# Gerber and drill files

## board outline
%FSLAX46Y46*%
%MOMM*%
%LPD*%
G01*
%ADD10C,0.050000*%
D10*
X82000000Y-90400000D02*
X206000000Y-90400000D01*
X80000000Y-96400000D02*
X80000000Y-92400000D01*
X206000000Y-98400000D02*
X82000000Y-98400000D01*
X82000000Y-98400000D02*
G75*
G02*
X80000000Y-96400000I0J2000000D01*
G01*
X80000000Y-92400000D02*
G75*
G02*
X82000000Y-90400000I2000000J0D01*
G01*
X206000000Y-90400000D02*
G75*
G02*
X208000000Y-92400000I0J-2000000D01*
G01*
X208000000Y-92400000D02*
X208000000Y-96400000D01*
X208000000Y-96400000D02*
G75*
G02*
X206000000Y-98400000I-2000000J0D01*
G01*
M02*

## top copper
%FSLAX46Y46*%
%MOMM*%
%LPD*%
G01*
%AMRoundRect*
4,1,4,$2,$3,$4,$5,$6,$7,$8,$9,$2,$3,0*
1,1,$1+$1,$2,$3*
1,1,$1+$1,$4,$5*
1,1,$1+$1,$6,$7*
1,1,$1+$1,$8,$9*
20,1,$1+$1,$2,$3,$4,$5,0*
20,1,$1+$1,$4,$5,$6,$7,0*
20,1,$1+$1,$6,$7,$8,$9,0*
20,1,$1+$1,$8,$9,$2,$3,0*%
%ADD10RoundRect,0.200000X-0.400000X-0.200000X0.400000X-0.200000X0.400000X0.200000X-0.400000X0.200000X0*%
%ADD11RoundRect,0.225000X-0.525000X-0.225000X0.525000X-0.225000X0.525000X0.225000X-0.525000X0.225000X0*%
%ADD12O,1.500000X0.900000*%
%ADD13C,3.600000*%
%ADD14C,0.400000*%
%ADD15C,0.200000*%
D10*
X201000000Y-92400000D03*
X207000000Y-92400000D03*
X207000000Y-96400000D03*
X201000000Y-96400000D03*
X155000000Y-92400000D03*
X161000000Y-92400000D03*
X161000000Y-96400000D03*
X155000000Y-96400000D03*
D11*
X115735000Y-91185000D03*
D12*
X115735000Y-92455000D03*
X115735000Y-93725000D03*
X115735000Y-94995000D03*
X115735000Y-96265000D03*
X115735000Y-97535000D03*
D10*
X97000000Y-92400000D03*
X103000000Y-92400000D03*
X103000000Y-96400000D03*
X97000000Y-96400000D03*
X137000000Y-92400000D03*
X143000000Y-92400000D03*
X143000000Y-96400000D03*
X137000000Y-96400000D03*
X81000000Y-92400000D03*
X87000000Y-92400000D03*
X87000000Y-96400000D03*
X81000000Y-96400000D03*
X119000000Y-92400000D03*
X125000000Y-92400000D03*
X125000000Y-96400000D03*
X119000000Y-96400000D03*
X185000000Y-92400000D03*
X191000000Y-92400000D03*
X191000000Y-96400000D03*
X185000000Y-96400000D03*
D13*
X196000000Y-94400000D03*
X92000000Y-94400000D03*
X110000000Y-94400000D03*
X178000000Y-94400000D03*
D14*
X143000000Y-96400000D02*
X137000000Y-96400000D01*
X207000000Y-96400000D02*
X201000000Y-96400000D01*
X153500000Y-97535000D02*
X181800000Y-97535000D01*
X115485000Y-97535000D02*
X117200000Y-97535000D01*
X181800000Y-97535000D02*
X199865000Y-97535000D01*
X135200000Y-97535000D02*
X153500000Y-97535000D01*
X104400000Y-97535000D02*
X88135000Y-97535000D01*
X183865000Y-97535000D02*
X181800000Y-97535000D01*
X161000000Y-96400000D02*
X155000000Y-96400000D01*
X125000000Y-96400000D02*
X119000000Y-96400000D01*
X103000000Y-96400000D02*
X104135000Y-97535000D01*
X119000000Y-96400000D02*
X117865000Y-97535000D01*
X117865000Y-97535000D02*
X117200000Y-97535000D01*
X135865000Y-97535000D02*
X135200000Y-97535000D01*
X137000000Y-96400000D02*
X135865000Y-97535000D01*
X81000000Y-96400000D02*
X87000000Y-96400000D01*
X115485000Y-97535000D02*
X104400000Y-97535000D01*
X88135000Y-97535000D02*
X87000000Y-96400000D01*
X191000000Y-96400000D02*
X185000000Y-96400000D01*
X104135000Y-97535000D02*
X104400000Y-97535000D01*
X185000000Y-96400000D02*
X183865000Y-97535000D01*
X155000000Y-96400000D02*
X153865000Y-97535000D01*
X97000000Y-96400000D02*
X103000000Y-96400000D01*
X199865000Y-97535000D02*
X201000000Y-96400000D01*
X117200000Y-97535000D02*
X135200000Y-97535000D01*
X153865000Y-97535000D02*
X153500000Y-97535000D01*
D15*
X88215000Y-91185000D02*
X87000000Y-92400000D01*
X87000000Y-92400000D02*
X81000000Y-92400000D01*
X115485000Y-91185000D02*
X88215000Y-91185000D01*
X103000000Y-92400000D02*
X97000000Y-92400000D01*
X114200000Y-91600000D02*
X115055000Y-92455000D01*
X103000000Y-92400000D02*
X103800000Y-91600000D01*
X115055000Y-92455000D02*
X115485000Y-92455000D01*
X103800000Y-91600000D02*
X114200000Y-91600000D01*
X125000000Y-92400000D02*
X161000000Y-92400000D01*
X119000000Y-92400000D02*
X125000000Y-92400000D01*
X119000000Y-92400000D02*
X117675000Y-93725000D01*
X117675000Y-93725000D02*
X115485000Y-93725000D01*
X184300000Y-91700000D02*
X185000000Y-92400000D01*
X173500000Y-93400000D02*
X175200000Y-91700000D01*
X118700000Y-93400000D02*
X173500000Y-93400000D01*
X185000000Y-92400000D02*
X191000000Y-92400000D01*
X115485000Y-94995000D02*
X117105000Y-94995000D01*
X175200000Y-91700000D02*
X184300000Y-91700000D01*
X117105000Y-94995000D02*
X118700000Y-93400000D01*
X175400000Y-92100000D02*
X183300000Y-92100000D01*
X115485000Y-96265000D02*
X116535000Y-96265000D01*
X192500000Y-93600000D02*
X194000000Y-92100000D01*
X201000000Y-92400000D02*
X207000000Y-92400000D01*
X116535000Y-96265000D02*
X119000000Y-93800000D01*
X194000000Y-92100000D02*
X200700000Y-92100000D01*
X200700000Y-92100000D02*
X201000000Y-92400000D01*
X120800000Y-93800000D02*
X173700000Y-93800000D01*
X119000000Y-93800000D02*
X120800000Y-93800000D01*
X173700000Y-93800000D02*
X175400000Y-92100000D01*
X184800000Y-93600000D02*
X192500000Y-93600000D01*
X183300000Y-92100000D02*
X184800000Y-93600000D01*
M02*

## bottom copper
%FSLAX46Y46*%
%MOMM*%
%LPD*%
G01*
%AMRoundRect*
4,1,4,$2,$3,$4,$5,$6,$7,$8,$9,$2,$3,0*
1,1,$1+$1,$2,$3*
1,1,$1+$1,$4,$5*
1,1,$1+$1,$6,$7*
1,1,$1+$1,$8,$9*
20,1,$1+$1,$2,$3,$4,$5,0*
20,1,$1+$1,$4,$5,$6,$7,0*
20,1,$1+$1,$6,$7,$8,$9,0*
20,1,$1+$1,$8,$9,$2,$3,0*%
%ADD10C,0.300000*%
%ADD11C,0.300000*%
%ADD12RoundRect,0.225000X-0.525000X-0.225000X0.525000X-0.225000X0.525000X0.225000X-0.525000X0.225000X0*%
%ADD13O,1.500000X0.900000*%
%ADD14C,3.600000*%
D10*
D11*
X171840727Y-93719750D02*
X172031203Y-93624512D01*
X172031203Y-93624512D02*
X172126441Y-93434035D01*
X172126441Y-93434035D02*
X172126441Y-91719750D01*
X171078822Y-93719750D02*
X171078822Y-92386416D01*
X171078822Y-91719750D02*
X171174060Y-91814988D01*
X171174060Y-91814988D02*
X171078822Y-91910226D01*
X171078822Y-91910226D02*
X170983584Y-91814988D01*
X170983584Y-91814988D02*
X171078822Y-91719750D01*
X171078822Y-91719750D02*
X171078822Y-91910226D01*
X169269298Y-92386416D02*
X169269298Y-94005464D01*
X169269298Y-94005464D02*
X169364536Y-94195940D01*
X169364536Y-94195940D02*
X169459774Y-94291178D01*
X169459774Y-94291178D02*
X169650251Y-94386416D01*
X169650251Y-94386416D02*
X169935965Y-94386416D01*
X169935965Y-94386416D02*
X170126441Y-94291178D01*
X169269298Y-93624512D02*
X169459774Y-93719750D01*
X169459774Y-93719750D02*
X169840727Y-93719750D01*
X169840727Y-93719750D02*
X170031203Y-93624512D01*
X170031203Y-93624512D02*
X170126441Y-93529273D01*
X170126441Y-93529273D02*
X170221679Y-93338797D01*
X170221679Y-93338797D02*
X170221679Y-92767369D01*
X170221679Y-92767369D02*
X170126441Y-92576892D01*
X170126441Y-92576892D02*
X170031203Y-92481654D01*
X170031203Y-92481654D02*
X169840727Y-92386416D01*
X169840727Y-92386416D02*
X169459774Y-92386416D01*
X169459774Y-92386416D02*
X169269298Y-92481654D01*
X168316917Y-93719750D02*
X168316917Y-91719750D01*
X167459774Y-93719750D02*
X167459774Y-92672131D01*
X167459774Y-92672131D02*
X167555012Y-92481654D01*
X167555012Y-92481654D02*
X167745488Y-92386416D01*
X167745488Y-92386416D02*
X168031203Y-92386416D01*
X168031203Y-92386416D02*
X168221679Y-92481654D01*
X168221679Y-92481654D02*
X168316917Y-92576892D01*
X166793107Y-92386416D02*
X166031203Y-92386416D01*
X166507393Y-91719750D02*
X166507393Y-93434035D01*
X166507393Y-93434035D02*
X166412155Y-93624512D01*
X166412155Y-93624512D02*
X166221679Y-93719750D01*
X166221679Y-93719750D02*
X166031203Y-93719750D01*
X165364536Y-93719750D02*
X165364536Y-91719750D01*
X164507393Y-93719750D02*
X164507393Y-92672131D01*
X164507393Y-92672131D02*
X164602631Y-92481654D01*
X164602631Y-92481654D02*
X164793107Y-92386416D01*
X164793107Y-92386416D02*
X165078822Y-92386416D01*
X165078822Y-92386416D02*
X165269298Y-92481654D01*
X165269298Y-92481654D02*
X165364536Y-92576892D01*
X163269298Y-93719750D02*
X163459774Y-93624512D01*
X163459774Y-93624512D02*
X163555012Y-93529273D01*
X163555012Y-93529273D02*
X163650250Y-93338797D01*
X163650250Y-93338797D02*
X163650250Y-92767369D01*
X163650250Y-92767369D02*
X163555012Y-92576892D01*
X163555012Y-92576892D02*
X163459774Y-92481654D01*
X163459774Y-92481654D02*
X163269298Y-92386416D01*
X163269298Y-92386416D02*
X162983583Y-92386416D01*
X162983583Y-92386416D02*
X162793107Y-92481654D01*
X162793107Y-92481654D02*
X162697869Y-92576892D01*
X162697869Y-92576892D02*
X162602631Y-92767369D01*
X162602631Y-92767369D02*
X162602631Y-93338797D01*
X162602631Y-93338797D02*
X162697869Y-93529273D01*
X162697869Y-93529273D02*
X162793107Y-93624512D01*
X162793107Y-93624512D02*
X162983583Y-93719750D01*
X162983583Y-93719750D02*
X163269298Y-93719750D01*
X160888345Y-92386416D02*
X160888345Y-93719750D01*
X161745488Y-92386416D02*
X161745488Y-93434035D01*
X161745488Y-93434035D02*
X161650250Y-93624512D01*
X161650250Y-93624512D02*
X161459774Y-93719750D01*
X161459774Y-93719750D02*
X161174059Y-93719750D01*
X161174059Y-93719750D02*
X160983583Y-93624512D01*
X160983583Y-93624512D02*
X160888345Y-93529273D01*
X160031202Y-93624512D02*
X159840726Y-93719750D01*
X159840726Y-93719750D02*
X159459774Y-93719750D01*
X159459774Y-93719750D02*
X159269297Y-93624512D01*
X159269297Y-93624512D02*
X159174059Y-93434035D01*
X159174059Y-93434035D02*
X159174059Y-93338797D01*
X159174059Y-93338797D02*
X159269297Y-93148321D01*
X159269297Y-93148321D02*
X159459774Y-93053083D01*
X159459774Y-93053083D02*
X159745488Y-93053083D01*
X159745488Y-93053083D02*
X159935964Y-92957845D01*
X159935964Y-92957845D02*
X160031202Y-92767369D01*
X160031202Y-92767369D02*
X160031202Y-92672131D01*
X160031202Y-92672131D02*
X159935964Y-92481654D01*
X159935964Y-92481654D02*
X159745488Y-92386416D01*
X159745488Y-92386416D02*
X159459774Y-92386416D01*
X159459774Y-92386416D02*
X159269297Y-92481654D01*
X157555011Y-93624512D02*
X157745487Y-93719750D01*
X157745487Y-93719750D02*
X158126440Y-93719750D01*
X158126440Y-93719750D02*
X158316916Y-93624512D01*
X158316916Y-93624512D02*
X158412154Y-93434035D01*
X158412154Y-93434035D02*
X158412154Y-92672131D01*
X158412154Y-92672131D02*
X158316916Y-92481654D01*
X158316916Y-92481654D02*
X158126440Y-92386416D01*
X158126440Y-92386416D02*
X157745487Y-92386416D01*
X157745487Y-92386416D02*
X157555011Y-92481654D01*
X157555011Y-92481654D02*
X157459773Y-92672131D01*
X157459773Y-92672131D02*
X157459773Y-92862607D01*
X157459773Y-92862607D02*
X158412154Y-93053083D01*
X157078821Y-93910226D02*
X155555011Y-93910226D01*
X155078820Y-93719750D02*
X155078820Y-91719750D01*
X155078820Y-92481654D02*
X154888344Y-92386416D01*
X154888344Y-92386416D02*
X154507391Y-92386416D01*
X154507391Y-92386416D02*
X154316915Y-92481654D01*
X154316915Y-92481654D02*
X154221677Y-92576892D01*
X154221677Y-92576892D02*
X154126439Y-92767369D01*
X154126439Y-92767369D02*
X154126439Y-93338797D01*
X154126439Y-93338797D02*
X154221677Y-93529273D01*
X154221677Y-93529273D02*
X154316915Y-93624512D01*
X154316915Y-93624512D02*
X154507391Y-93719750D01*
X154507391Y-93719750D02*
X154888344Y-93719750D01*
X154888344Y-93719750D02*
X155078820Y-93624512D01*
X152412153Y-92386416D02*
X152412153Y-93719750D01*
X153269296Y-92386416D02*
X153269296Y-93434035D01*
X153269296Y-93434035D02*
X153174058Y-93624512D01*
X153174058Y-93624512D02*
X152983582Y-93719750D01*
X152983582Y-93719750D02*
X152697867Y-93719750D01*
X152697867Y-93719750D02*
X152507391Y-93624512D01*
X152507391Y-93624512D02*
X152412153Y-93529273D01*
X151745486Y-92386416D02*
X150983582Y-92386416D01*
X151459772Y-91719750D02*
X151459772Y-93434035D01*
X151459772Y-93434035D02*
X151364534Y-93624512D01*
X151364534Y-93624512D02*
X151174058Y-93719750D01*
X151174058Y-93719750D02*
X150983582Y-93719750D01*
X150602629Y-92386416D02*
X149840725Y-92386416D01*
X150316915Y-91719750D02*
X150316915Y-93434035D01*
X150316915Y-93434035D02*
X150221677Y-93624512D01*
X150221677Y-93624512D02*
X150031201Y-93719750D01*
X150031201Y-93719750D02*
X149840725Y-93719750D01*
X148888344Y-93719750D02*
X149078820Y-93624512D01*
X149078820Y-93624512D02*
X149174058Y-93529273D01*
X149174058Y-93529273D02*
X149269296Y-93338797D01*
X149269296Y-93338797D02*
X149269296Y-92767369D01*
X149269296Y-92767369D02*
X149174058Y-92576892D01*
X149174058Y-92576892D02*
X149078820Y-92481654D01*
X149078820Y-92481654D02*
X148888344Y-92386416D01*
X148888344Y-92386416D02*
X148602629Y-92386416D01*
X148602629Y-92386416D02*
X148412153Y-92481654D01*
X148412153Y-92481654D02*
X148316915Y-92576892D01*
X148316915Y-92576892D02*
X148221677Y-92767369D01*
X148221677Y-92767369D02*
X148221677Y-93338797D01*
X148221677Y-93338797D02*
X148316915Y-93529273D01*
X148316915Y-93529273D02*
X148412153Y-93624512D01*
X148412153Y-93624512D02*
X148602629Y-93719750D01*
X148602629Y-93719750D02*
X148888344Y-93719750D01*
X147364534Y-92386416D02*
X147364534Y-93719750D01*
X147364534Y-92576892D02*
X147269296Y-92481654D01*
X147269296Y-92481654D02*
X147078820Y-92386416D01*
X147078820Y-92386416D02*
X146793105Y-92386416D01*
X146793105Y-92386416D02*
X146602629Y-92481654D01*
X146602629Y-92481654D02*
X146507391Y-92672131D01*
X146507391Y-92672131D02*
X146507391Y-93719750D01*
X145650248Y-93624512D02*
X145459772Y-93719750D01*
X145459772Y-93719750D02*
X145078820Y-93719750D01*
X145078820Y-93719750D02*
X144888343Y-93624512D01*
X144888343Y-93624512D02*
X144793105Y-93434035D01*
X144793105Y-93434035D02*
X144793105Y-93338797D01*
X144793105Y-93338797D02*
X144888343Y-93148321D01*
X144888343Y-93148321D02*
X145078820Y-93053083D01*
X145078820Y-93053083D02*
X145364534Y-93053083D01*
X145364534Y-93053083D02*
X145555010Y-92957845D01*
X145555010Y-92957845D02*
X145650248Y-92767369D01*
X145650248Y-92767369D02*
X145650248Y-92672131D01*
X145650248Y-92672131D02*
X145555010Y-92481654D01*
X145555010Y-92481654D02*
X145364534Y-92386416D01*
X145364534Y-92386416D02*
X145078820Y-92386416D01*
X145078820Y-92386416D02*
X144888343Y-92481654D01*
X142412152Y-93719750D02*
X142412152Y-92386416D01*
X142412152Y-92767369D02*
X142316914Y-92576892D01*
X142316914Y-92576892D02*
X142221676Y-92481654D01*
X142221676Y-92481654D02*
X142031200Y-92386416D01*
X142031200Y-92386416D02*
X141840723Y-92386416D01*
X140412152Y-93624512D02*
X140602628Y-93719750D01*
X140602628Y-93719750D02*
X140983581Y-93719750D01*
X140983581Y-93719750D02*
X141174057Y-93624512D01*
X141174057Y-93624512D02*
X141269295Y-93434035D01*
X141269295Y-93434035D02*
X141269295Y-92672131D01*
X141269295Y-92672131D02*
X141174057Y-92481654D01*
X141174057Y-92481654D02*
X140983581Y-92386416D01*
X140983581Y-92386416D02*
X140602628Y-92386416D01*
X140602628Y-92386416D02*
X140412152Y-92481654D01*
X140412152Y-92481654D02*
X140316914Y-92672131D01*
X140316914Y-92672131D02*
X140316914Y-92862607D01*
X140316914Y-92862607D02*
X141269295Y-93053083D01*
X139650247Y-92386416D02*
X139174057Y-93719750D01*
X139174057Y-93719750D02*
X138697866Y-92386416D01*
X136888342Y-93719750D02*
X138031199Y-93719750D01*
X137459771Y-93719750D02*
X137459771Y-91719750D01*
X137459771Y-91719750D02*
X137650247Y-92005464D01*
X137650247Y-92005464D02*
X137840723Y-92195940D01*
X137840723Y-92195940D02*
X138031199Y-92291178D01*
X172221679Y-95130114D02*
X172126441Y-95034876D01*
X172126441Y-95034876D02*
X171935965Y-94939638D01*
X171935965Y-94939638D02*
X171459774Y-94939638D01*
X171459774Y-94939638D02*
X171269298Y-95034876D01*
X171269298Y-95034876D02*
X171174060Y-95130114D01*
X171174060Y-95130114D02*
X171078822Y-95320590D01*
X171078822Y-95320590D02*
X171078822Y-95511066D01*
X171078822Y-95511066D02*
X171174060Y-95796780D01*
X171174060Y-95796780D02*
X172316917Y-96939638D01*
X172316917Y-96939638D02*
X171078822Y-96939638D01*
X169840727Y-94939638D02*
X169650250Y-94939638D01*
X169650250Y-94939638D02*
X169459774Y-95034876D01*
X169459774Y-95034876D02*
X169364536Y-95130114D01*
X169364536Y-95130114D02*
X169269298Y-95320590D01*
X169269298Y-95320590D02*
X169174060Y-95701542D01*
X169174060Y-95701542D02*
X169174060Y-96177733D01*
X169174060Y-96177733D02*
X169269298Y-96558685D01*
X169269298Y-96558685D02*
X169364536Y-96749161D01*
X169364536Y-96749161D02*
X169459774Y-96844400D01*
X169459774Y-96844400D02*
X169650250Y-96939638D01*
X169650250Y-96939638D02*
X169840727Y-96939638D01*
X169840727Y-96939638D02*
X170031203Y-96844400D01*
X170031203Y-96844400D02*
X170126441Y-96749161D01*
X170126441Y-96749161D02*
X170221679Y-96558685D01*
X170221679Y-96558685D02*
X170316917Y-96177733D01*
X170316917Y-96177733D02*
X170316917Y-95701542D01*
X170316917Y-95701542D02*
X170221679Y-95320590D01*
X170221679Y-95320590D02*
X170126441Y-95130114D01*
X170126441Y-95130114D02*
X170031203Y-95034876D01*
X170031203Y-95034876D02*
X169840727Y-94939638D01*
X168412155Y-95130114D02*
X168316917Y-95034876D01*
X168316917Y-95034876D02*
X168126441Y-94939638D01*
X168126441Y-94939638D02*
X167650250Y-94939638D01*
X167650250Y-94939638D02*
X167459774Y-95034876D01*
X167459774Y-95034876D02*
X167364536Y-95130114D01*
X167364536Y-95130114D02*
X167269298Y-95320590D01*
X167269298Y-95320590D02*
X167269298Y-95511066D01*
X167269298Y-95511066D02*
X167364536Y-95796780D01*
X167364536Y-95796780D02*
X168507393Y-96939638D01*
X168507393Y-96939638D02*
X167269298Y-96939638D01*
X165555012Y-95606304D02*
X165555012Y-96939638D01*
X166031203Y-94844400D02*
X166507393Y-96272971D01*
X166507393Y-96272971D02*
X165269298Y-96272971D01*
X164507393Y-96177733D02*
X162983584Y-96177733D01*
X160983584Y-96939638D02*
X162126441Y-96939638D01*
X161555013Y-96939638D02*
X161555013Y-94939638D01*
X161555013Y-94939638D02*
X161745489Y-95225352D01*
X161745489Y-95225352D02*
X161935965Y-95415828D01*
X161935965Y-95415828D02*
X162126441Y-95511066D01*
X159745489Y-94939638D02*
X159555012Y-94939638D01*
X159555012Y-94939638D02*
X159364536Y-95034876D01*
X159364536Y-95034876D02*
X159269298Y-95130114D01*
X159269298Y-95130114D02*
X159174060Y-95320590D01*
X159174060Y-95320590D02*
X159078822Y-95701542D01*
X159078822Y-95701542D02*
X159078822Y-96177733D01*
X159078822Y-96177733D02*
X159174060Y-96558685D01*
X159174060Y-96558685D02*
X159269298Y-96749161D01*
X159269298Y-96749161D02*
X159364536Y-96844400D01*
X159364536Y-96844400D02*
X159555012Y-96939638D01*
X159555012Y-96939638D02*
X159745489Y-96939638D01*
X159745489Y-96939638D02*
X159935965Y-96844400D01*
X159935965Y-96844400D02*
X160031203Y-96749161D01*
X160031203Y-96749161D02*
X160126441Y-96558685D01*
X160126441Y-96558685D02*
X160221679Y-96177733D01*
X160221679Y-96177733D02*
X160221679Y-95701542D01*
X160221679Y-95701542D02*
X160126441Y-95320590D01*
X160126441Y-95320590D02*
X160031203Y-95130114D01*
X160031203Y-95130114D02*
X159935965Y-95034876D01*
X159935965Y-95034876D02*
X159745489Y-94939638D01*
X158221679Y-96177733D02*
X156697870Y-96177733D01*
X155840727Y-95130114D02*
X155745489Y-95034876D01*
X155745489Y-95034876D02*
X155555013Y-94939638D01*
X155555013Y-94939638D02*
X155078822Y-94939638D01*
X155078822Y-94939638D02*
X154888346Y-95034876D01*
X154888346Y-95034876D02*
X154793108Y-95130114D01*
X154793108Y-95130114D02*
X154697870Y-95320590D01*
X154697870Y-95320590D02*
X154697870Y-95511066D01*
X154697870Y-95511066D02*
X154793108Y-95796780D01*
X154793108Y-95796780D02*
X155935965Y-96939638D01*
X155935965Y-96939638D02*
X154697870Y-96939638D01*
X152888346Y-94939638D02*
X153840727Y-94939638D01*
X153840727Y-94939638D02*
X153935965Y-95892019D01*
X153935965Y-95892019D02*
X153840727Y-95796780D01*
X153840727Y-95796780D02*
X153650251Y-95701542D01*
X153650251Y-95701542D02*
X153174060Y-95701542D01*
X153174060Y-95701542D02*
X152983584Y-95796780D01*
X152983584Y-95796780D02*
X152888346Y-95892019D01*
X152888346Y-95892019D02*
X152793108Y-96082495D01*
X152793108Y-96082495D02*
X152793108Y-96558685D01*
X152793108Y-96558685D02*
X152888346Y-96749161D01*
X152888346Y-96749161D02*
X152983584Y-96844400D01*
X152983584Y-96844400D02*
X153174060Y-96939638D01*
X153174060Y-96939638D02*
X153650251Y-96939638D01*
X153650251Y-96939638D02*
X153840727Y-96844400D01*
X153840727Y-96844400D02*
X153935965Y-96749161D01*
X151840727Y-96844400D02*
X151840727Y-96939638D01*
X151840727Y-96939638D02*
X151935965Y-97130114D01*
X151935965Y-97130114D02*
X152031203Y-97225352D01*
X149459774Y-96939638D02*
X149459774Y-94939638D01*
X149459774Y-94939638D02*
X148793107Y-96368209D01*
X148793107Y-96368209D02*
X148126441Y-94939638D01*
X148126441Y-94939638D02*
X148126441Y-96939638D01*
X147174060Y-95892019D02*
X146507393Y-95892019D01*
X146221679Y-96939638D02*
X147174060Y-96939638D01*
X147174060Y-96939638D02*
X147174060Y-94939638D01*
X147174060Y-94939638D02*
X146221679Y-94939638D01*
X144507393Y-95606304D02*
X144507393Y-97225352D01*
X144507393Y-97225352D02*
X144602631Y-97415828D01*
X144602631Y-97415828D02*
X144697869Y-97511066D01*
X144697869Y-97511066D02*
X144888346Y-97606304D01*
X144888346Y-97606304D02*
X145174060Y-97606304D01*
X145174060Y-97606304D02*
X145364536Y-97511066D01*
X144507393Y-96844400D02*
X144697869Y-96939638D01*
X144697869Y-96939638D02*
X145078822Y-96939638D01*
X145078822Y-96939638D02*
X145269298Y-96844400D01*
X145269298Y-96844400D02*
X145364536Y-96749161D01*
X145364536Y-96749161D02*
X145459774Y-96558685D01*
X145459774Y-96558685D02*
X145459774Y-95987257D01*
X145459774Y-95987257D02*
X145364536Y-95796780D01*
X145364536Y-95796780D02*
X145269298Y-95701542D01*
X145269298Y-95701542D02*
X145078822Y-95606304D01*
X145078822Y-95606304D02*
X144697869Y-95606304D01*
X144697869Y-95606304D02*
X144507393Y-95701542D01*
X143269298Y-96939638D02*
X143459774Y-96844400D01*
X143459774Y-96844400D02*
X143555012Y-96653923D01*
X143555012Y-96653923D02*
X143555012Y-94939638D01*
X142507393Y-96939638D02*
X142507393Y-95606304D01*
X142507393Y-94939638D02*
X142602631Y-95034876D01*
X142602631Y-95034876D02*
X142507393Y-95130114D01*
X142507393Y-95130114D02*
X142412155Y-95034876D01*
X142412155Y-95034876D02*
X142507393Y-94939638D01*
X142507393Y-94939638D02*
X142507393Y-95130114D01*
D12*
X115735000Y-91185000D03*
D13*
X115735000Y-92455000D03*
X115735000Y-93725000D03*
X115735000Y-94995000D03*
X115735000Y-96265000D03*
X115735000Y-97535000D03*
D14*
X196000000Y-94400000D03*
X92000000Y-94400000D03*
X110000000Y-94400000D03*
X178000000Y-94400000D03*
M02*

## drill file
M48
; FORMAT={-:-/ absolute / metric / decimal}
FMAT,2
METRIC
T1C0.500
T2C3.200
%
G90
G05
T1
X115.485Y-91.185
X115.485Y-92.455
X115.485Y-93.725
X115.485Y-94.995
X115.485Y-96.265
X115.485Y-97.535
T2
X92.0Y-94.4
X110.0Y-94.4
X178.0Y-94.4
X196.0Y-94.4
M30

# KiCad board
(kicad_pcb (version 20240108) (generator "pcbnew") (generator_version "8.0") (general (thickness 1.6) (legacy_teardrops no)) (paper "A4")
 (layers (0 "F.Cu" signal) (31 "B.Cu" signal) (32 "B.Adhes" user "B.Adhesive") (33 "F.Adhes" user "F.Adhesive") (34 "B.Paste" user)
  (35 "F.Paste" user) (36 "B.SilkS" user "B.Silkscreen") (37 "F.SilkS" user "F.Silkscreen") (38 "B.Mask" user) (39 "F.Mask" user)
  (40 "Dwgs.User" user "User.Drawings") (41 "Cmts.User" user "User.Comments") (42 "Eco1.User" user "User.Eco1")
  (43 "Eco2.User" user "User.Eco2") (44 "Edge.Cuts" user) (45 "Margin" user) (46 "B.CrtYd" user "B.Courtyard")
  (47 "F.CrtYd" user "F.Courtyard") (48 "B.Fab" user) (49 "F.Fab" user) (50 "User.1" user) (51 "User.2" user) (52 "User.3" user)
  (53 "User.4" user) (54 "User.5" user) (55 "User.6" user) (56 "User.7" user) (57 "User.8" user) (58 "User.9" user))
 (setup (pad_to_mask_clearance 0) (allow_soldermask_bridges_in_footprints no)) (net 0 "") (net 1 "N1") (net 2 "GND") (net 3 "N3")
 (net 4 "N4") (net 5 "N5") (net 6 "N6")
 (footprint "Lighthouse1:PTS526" (layer "F.Cu") (at 204 94.4)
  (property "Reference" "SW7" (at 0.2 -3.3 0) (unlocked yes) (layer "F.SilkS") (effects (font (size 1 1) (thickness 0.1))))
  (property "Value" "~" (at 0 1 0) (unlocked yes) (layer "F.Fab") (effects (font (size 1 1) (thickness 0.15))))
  (pad "1" smd roundrect (at -3 -2) (size 1.2 0.8) (layers "F.Cu" "F.Paste" "F.Mask") (roundrect_rratio 0.25) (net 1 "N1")
   (thermal_bridge_angle 45))
  (pad "2" smd roundrect (at 3 -2) (size 1.2 0.8) (layers "F.Cu" "F.Paste" "F.Mask") (roundrect_rratio 0.25) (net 1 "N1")
   (thermal_bridge_angle 45))
  (pad "3" smd roundrect (at 3 2) (size 1.2 0.8) (layers "F.Cu" "F.Paste" "F.Mask") (roundrect_rratio 0.25) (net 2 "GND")
   (thermal_bridge_angle 45))
  (pad "4" smd roundrect (at -3 2) (size 1.2 0.8) (layers "F.Cu" "F.Paste" "F.Mask") (roundrect_rratio 0.25) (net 2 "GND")
   (thermal_bridge_angle 45)))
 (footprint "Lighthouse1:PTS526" (layer "F.Cu") (at 158 94.4)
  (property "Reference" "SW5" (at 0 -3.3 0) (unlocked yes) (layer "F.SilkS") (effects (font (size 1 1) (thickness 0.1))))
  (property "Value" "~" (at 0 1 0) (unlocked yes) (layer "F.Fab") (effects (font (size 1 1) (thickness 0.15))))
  (pad "1" smd roundrect (at -3 -2) (size 1.2 0.8) (layers "F.Cu" "F.Paste" "F.Mask") (roundrect_rratio 0.25) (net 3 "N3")
   (thermal_bridge_angle 45))
  (pad "2" smd roundrect (at 3 -2) (size 1.2 0.8) (layers "F.Cu" "F.Paste" "F.Mask") (roundrect_rratio 0.25) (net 3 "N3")
   (thermal_bridge_angle 45))
  (pad "3" smd roundrect (at 3 2) (size 1.2 0.8) (layers "F.Cu" "F.Paste" "F.Mask") (roundrect_rratio 0.25) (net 2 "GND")
   (thermal_bridge_angle 45))
  (pad "4" smd roundrect (at -3 2) (size 1.2 0.8) (layers "F.Cu" "F.Paste" "F.Mask") (roundrect_rratio 0.25) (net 2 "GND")
   (thermal_bridge_angle 45)))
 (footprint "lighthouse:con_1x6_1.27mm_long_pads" (layer "F.Cu") (at 115.485 91.185)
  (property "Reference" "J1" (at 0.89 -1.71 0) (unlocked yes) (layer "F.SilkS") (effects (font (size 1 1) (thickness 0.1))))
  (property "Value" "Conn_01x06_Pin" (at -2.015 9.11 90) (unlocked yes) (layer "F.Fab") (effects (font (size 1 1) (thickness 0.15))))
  (pad "1" thru_hole roundrect (at 0 0) (size 1.5 0.9) (drill 0.5 (offset 0.25 0)) (layers "*.Cu" "*.Mask") (remove_unused_layers no)
   (roundrect_rratio 0.25) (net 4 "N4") (thermal_bridge_angle 45))
  (pad "2" thru_hole oval (at 0 1.27) (size 1.5 0.9) (drill 0.5 (offset 0.25 0)) (layers "*.Cu" "*.Mask") (remove_unused_layers no)
   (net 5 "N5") (thermal_bridge_angle 45))
  (pad "3" thru_hole oval (at 0 2.54) (size 1.5 0.9) (drill 0.5 (offset 0.25 0)) (layers "*.Cu" "*.Mask") (remove_unused_layers no)
   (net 3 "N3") (thermal_bridge_angle 45))
  (pad "4" thru_hole oval (at 0 3.81) (size 1.5 0.9) (drill 0.5 (offset 0.25 0)) (layers "*.Cu" "*.Mask") (remove_unused_layers no)
   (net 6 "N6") (thermal_bridge_angle 45))
  (pad "5" thru_hole oval (at 0 5.08) (size 1.5 0.9) (drill 0.5 (offset 0.25 0)) (layers "*.Cu" "*.Mask") (remove_unused_layers no)
   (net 1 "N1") (thermal_bridge_angle 45))
  (pad "6" thru_hole oval (at 0 6.35) (size 1.5 0.9) (drill 0.5 (offset 0.25 0)) (layers "*.Cu" "*.Mask") (remove_unused_layers no)
   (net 2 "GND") (thermal_bridge_angle 45)))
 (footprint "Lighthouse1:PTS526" (layer "F.Cu") (at 100 94.4)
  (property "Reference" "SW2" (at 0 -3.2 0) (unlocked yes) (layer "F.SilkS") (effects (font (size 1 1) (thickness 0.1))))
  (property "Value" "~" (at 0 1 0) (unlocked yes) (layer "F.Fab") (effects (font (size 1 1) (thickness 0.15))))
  (pad "1" smd roundrect (at -3 -2) (size 1.2 0.8) (layers "F.Cu" "F.Paste" "F.Mask") (roundrect_rratio 0.25) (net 5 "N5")
   (thermal_bridge_angle 45))
  (pad "2" smd roundrect (at 3 -2) (size 1.2 0.8) (layers "F.Cu" "F.Paste" "F.Mask") (roundrect_rratio 0.25) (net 5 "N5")
   (thermal_bridge_angle 45))
  (pad "3" smd roundrect (at 3 2) (size 1.2 0.8) (layers "F.Cu" "F.Paste" "F.Mask") (roundrect_rratio 0.25) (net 2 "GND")
   (thermal_bridge_angle 45))
  (pad "4" smd roundrect (at -3 2) (size 1.2 0.8) (layers "F.Cu" "F.Paste" "F.Mask") (roundrect_rratio 0.25) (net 2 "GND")
   (thermal_bridge_angle 45)))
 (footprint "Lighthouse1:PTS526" (layer "F.Cu") (at 140 94.4)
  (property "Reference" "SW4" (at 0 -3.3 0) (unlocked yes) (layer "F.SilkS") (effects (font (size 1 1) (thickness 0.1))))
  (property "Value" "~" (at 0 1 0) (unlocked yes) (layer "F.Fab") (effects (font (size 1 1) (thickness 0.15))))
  (pad "1" smd roundrect (at -3 -2) (size 1.2 0.8) (layers "F.Cu" "F.Paste" "F.Mask") (roundrect_rratio 0.25) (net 3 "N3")
   (thermal_bridge_angle 45))
  (pad "2" smd roundrect (at 3 -2) (size 1.2 0.8) (layers "F.Cu" "F.Paste" "F.Mask") (roundrect_rratio 0.25) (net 3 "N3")
   (thermal_bridge_angle 45))
  (pad "3" smd roundrect (at 3 2) (size 1.2 0.8) (layers "F.Cu" "F.Paste" "F.Mask") (roundrect_rratio 0.25) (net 2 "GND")
   (thermal_bridge_angle 45))
  (pad "4" smd roundrect (at -3 2) (size 1.2 0.8) (layers "F.Cu" "F.Paste" "F.Mask") (roundrect_rratio 0.25) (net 2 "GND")
   (thermal_bridge_angle 45)))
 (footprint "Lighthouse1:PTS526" (layer "F.Cu") (at 84 94.4)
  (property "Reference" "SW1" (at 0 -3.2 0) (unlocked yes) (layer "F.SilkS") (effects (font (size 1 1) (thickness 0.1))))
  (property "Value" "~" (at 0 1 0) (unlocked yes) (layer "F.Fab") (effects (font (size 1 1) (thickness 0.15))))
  (pad "1" smd roundrect (at -3 -2) (size 1.2 0.8) (layers "F.Cu" "F.Paste" "F.Mask") (roundrect_rratio 0.25) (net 4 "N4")
   (thermal_bridge_angle 45))
  (pad "2" smd roundrect (at 3 -2) (size 1.2 0.8) (layers "F.Cu" "F.Paste" "F.Mask") (roundrect_rratio 0.25) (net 4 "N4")
   (thermal_bridge_angle 45))
  (pad "3" smd roundrect (at 3 2) (size 1.2 0.8) (layers "F.Cu" "F.Paste" "F.Mask") (roundrect_rratio 0.25) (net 2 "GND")
   (thermal_bridge_angle 45))
  (pad "4" smd roundrect (at -3 2) (size 1.2 0.8) (layers "F.Cu" "F.Paste" "F.Mask") (roundrect_rratio 0.25) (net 2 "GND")
   (thermal_bridge_angle 45)))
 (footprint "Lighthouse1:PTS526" (layer "F.Cu") (at 122 94.4)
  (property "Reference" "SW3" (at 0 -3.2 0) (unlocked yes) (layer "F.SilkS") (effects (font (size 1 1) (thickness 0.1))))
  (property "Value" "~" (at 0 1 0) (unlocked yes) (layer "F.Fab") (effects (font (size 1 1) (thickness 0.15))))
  (pad "1" smd roundrect (at -3 -2) (size 1.2 0.8) (layers "F.Cu" "F.Paste" "F.Mask") (roundrect_rratio 0.25) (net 3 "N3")
   (thermal_bridge_angle 45))
  (pad "2" smd roundrect (at 3 -2) (size 1.2 0.8) (layers "F.Cu" "F.Paste" "F.Mask") (roundrect_rratio 0.25) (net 3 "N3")
   (thermal_bridge_angle 45))
  (pad "3" smd roundrect (at 3 2) (size 1.2 0.8) (layers "F.Cu" "F.Paste" "F.Mask") (roundrect_rratio 0.25) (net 2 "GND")
   (thermal_bridge_angle 45))
  (pad "4" smd roundrect (at -3 2) (size 1.2 0.8) (layers "F.Cu" "F.Paste" "F.Mask") (roundrect_rratio 0.25) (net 2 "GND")
   (thermal_bridge_angle 45)))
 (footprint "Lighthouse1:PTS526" (layer "F.Cu") (at 188 94.4)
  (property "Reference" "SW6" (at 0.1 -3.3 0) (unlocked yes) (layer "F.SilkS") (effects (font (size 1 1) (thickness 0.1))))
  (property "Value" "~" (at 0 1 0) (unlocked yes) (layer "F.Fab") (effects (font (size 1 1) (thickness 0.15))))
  (pad "1" smd roundrect (at -3 -2) (size 1.2 0.8) (layers "F.Cu" "F.Paste" "F.Mask") (roundrect_rratio 0.25) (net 6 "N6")
   (thermal_bridge_angle 45))
  (pad "2" smd roundrect (at 3 -2) (size 1.2 0.8) (layers "F.Cu" "F.Paste" "F.Mask") (roundrect_rratio 0.25) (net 6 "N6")
   (thermal_bridge_angle 45))
  (pad "3" smd roundrect (at 3 2) (size 1.2 0.8) (layers "F.Cu" "F.Paste" "F.Mask") (roundrect_rratio 0.25) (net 2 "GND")
   (thermal_bridge_angle 45))
  (pad "4" smd roundrect (at -3 2) (size 1.2 0.8) (layers "F.Cu" "F.Paste" "F.Mask") (roundrect_rratio 0.25) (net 2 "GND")
   (thermal_bridge_angle 45)))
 (gr_line (start 82 90.4) (end 206 90.4) (stroke (width 0.05) (type default)) (layer "Edge.Cuts"))
 (gr_line (start 80 96.4) (end 80 92.4) (stroke (width 0.05) (type default)) (layer "Edge.Cuts"))
 (gr_line (start 206 98.4) (end 82 98.4) (stroke (width 0.05) (type default)) (layer "Edge.Cuts"))
 (gr_arc (start 82 98.4) (mid 80.585786 97.814214) (end 80 96.4) (stroke (width 0.05) (type default)) (layer "Edge.Cuts"))
 (gr_arc (start 80 92.4) (mid 80.585786 90.985786) (end 82 90.4) (stroke (width 0.05) (type default)) (layer "Edge.Cuts"))
 (gr_arc (start 206 90.4) (mid 207.414214 90.985786) (end 208 92.4) (stroke (width 0.05) (type default)) (layer "Edge.Cuts"))
 (gr_line (start 208 92.4) (end 208 96.4) (stroke (width 0.05) (type default)) (layer "Edge.Cuts"))
 (gr_arc (start 208 96.4) (mid 207.414214 97.814214) (end 206 98.4) (stroke (width 0.05) (type default)) (layer "Edge.Cuts"))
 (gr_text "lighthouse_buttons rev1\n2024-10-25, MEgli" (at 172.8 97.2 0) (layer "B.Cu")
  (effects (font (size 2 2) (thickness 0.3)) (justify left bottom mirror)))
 (via (at 196 94.4) (size 3.6) (drill 3.2) (layers "F.Cu" "B.Cu") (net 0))
 (via (at 92 94.4) (size 3.6) (drill 3.2) (layers "F.Cu" "B.Cu") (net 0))
 (via (at 110 94.4) (size 3.6) (drill 3.2) (layers "F.Cu" "B.Cu") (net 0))
 (via (at 178 94.4) (size 3.6) (drill 3.2) (layers "F.Cu" "B.Cu") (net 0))
 (segment (start 143 96.4) (end 137 96.4) (width 0.4) (layer "F.Cu") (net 2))
 (segment (start 207 96.4) (end 201 96.4) (width 0.4) (layer "F.Cu") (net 2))
 (segment (start 153.5 97.535) (end 181.8 97.535) (width 0.4) (layer "F.Cu") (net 2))
 (segment (start 115.485 97.535) (end 117.2 97.535) (width 0.4) (layer "F.Cu") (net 2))
 (segment (start 181.8 97.535) (end 199.865 97.535) (width 0.4) (layer "F.Cu") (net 2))
 (segment (start 135.2 97.535) (end 153.5 97.535) (width 0.4) (layer "F.Cu") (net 2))
 (segment (start 104.4 97.535) (end 88.135 97.535) (width 0.4) (layer "F.Cu") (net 2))
 (segment (start 183.865 97.535) (end 181.8 97.535) (width 0.4) (layer "F.Cu") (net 2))
 (segment (start 161 96.4) (end 155 96.4) (width 0.4) (layer "F.Cu") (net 2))
 (segment (start 125 96.4) (end 119 96.4) (width 0.4) (layer "F.Cu") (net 2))
 (segment (start 103 96.4) (end 104.135 97.535) (width 0.4) (layer "F.Cu") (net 2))
 (segment (start 119 96.4) (end 117.865 97.535) (width 0.4) (layer "F.Cu") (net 2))
 (segment (start 117.865 97.535) (end 117.2 97.535) (width 0.4) (layer "F.Cu") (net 2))
 (segment (start 135.865 97.535) (end 135.2 97.535) (width 0.4) (layer "F.Cu") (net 2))
 (segment (start 137 96.4) (end 135.865 97.535) (width 0.4) (layer "F.Cu") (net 2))
 (segment (start 81 96.4) (end 87 96.4) (width 0.4) (layer "F.Cu") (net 2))
 (segment (start 115.485 97.535) (end 104.4 97.535) (width 0.4) (layer "F.Cu") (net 2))
 (segment (start 88.135 97.535) (end 87 96.4) (width 0.4) (layer "F.Cu") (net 2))
 (segment (start 191 96.4) (end 185 96.4) (width 0.4) (layer "F.Cu") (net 2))
 (segment (start 104.135 97.535) (end 104.4 97.535) (width 0.4) (layer "F.Cu") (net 2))
 (segment (start 185 96.4) (end 183.865 97.535) (width 0.4) (layer "F.Cu") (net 2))
 (segment (start 155 96.4) (end 153.865 97.535) (width 0.4) (layer "F.Cu") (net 2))
 (segment (start 97 96.4) (end 103 96.4) (width 0.4) (layer "F.Cu") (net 2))
 (segment (start 199.865 97.535) (end 201 96.4) (width 0.4) (layer "F.Cu") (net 2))
 (segment (start 117.2 97.535) (end 135.2 97.535) (width 0.4) (layer "F.Cu") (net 2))
 (segment (start 153.865 97.535) (end 153.5 97.535) (width 0.4) (layer "F.Cu") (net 2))
 (segment (start 88.215 91.185) (end 87 92.4) (width 0.2) (layer "F.Cu") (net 4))
 (segment (start 87 92.4) (end 81 92.4) (width 0.2) (layer "F.Cu") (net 4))
 (segment (start 115.485 91.185) (end 88.215 91.185) (width 0.2) (layer "F.Cu") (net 4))
 (segment (start 103 92.4) (end 97 92.4) (width 0.2) (layer "F.Cu") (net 5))
 (segment (start 114.2 91.6) (end 115.055 92.455) (width 0.2) (layer "F.Cu") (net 5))
 (segment (start 103 92.4) (end 103.8 91.6) (width 0.2) (layer "F.Cu") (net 5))
 (segment (start 115.055 92.455) (end 115.485 92.455) (width 0.2) (layer "F.Cu") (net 5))
 (segment (start 103.8 91.6) (end 114.2 91.6) (width 0.2) (layer "F.Cu") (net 5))
 (segment (start 125 92.4) (end 161 92.4) (width 0.2) (layer "F.Cu") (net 3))
 (segment (start 119 92.4) (end 125 92.4) (width 0.2) (layer "F.Cu") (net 3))
 (segment (start 119 92.4) (end 117.675 93.725) (width 0.2) (layer "F.Cu") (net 3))
 (segment (start 117.675 93.725) (end 115.485 93.725) (width 0.2) (layer "F.Cu") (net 3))
 (segment (start 184.3 91.7) (end 185 92.4) (width 0.2) (layer "F.Cu") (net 6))
 (segment (start 173.5 93.4) (end 175.2 91.7) (width 0.2) (layer "F.Cu") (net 6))
 (segment (start 118.7 93.4) (end 173.5 93.4) (width 0.2) (layer "F.Cu") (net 6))
 (segment (start 185 92.4) (end 191 92.4) (width 0.2) (layer "F.Cu") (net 6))
 (segment (start 115.485 94.995) (end 117.105 94.995) (width 0.2) (layer "F.Cu") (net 6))
 (segment (start 175.2 91.7) (end 184.3 91.7) (width 0.2) (layer "F.Cu") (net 6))
 (segment (start 117.105 94.995) (end 118.7 93.4) (width 0.2) (layer "F.Cu") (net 6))
 (segment (start 175.4 92.1) (end 183.3 92.1) (width 0.2) (layer "F.Cu") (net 1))
 (segment (start 115.485 96.265) (end 116.535 96.265) (width 0.2) (layer "F.Cu") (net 1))
 (segment (start 192.5 93.6) (end 194 92.1) (width 0.2) (layer "F.Cu") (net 1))
 (segment (start 201 92.4) (end 207 92.4) (width 0.2) (layer "F.Cu") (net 1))
 (segment (start 116.535 96.265) (end 119 93.8) (width 0.2) (layer "F.Cu") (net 1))
 (segment (start 194 92.1) (end 200.7 92.1) (width 0.2) (layer "F.Cu") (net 1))
 (segment (start 200.7 92.1) (end 201 92.4) (width 0.2) (layer "F.Cu") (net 1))
 (segment (start 120.8 93.8) (end 173.7 93.8) (width 0.2) (layer "F.Cu") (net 1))
 (segment (start 119 93.8) (end 120.8 93.8) (width 0.2) (layer "F.Cu") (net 1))
 (segment (start 173.7 93.8) (end 175.4 92.1) (width 0.2) (layer "F.Cu") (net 1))
 (segment (start 184.8 93.6) (end 192.5 93.6) (width 0.2) (layer "F.Cu") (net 1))
 (segment (start 183.3 92.1) (end 184.8 93.6) (width 0.2) (layer "F.Cu") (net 1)))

